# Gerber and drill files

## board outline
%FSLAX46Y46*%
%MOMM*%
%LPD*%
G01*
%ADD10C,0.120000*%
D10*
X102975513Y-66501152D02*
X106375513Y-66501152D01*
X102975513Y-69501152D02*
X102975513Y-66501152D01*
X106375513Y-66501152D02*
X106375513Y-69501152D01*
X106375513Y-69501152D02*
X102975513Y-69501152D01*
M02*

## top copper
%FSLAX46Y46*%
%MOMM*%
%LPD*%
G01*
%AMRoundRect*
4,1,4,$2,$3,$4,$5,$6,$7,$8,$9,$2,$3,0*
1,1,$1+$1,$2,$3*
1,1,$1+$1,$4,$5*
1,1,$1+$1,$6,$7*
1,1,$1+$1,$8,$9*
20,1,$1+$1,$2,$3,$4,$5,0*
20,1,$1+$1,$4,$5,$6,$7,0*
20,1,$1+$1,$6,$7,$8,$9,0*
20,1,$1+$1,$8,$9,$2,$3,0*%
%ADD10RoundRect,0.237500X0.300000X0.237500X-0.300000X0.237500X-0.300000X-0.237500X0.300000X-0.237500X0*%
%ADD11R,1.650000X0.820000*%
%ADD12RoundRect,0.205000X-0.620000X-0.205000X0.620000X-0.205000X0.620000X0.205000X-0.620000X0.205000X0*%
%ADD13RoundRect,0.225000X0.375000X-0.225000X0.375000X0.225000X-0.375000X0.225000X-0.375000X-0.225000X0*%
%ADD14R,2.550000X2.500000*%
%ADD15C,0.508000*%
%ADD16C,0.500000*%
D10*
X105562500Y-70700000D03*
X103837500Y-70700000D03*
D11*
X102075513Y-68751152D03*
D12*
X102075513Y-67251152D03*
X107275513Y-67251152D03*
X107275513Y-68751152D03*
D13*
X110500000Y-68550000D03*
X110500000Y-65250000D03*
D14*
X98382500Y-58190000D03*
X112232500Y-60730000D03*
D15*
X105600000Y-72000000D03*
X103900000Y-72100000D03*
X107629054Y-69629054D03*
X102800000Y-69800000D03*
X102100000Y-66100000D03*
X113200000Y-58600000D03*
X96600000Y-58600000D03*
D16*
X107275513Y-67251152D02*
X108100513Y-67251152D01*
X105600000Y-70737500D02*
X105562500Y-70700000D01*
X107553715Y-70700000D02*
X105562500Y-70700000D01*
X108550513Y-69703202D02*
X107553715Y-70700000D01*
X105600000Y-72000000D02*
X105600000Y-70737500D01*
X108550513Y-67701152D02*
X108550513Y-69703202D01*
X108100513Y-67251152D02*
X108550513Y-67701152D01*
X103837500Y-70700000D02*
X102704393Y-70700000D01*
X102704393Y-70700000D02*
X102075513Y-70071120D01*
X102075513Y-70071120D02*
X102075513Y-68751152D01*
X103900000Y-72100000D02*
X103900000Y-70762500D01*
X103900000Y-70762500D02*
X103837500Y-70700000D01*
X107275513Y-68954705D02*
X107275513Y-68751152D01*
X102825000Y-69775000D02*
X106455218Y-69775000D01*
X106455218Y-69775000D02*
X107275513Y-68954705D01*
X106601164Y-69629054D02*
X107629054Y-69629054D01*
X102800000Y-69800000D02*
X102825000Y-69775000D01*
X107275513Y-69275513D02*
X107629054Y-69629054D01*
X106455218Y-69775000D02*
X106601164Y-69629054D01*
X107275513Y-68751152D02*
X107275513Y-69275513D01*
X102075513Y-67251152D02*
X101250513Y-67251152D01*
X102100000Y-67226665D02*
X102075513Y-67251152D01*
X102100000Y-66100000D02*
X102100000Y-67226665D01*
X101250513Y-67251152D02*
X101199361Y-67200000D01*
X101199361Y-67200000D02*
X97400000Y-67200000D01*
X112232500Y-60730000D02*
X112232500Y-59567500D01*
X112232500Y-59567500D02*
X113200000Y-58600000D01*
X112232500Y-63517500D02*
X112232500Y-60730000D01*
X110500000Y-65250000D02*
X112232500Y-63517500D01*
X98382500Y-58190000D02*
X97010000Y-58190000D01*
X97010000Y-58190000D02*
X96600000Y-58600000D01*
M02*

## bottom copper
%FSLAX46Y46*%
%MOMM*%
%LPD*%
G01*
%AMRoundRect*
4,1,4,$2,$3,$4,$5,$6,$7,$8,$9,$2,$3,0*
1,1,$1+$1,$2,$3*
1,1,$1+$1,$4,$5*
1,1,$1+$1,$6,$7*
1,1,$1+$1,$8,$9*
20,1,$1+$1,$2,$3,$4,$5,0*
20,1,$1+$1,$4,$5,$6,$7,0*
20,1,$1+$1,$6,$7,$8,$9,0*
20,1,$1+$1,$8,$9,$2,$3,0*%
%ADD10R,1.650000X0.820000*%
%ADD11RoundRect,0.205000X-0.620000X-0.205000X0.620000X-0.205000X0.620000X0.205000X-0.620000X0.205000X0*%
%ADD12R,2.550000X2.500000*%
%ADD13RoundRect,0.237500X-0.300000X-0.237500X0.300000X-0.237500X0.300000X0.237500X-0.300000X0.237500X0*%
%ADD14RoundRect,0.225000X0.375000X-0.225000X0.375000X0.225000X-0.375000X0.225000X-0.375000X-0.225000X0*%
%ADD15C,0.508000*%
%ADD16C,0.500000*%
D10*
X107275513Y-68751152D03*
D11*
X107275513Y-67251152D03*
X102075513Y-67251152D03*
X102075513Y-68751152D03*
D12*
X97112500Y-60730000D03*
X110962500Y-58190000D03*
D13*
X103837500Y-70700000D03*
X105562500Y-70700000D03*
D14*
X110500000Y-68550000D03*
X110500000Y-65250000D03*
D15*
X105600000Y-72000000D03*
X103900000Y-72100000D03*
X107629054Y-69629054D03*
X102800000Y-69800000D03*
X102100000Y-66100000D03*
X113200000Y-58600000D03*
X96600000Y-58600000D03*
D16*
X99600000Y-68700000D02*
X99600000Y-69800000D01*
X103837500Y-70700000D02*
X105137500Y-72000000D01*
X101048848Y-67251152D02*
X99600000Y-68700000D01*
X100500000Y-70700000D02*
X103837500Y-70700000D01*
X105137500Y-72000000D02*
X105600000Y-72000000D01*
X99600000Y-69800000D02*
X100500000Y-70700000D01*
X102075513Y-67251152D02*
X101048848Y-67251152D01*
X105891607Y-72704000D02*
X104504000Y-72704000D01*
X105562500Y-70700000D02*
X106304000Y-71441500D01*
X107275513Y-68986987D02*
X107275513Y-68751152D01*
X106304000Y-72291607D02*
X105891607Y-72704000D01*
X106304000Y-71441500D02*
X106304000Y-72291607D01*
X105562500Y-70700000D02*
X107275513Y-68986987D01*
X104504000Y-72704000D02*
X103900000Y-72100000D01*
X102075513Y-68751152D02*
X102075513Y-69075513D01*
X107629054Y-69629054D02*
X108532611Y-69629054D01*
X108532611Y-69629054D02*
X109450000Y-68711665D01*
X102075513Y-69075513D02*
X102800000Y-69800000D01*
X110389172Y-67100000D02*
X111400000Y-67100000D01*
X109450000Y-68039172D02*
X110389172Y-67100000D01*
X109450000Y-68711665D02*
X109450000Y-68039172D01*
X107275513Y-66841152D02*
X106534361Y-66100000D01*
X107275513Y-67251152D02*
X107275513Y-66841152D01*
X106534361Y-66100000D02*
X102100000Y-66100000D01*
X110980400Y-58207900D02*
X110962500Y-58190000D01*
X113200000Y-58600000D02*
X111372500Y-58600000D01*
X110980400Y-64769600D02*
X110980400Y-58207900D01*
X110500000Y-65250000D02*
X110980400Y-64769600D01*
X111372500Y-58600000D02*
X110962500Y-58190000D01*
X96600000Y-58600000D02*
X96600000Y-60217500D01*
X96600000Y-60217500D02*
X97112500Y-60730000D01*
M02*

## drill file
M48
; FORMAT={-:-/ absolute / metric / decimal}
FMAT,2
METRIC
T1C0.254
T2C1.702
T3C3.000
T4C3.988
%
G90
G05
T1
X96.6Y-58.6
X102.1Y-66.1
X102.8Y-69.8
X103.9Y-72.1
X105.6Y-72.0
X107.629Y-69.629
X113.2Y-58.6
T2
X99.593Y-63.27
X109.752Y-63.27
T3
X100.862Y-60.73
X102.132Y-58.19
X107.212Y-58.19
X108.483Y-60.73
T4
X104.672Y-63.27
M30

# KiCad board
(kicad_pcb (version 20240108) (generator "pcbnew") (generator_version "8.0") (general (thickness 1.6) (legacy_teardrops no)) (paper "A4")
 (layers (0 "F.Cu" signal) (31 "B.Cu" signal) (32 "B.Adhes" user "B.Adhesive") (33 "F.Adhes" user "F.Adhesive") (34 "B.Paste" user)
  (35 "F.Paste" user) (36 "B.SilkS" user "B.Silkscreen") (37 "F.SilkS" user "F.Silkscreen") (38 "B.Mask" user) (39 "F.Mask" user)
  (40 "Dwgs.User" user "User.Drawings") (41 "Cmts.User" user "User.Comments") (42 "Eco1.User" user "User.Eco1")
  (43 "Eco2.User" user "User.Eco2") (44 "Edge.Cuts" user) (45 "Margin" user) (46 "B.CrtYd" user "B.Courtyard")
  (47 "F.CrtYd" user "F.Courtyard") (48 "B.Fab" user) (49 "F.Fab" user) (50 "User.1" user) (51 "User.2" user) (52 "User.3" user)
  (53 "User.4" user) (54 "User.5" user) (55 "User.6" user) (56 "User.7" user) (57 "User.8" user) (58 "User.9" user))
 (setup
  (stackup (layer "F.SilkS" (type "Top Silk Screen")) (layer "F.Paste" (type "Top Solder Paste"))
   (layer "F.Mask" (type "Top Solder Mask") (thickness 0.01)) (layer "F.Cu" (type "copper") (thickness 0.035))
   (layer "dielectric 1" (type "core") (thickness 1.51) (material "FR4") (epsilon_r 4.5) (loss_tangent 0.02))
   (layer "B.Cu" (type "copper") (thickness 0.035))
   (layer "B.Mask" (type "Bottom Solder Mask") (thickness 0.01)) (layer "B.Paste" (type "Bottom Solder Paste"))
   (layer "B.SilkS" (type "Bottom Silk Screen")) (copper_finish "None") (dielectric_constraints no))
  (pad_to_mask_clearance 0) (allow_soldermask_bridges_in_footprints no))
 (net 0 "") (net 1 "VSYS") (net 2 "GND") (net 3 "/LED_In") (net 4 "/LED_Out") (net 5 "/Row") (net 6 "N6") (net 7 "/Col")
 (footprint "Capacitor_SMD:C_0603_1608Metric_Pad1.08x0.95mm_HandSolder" (layer "F.Cu") (at 104.7 70.7 180)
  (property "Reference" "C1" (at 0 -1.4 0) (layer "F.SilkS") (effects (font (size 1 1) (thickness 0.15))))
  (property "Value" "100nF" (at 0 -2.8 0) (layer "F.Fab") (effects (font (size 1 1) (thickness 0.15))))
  (pad "1" smd roundrect (at -0.8625 0 180) (size 1.075 0.95) (layers "F.Cu" "F.Paste" "F.Mask") (roundrect_rratio 0.25) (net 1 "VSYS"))
  (pad "2" smd roundrect (at 0.8625 0 180) (size 1.075 0.95) (layers "F.Cu" "F.Paste" "F.Mask") (roundrect_rratio 0.25) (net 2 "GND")))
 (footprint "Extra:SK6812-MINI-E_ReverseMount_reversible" (layer "F.Cu") (at 104.675513 68.001152)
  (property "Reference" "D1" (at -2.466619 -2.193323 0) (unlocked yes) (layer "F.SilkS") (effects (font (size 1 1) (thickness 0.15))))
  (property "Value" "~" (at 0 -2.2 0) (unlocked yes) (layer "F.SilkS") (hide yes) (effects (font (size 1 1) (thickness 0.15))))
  (fp_line (start -1.7 -1.5) (end 1.7 -1.5) (stroke (width 0.12) (type solid)) (layer "Edge.Cuts"))
  (fp_line (start -1.7 1.5) (end -1.7 -1.5) (stroke (width 0.12) (type solid)) (layer "Edge.Cuts"))
  (fp_line (start 1.7 -1.5) (end 1.7 1.5) (stroke (width 0.12) (type solid)) (layer "Edge.Cuts"))
  (fp_line (start 1.7 1.5) (end -1.7 1.5) (stroke (width 0.12) (type solid)) (layer "Edge.Cuts"))
  (pad "1" smd rect (at -2.6 0.75) (size 1.65 0.82) (layers "F.Cu" "F.Paste" "F.Mask") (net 2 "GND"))
  (pad "1" smd rect (at 2.6 0.75) (size 1.65 0.82) (layers "B.Cu" "B.Paste" "B.Mask") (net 2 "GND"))
  (pad "2" smd roundrect (at -2.6 -0.75) (size 1.65 0.82) (layers "F.Cu" "F.Paste" "F.Mask") (roundrect_rratio 0.25) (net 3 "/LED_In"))
  (pad "2" smd roundrect (at 2.6 -0.75) (size 1.65 0.82) (layers "B.Cu" "B.Paste" "B.Mask") (roundrect_rratio 0.25) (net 3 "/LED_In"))
  (pad "3" smd roundrect (at -2.6 -0.75) (size 1.65 0.82) (layers "B.Cu" "B.Paste" "B.Mask") (roundrect_rratio 0.25) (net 1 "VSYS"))
  (pad "3" smd roundrect (at 2.6 -0.75) (size 1.65 0.82) (layers "F.Cu" "F.Paste" "F.Mask") (roundrect_rratio 0.25) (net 1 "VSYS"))
  (pad "4" smd roundrect (at -2.6 0.75) (size 1.65 0.82) (layers "B.Cu" "B.Paste" "B.Mask") (roundrect_rratio 0.25) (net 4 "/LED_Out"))
  (pad "4" smd roundrect (at 2.6 0.75) (size 1.65 0.82) (layers "F.Cu" "F.Paste" "F.Mask") (roundrect_rratio 0.25) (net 4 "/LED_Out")))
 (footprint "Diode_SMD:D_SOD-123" (layer "F.Cu") (at 110.5 66.9 90)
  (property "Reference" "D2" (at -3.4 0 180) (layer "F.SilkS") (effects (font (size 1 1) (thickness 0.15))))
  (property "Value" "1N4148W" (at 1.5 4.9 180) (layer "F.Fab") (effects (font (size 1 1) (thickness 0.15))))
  (pad "1" smd roundrect (at -1.65 0 90) (size 0.9 1.2) (layers "F.Cu" "F.Paste" "F.Mask") (roundrect_rratio 0.25) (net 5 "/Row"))
  (pad "2" smd roundrect (at 1.65 0 90) (size 0.9 1.2) (layers "F.Cu" "F.Paste" "F.Mask") (roundrect_rratio 0.25) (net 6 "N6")))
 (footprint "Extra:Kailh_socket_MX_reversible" (layer "F.Cu") (at 104.6725 63.27)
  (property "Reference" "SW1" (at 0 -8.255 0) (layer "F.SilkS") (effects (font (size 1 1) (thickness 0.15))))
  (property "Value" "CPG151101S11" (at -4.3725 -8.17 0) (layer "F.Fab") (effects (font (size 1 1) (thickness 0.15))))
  (pad "" np_thru_hole circle (at -5.08 0) (size 1.7018 1.7018) (drill 1.7018) (layers "*.Cu" "*.Mask"))
  (pad "" np_thru_hole circle (at -3.81 -2.54) (size 3 3) (drill 3) (layers "*.Cu" "*.Mask"))
  (pad "" np_thru_hole circle (at -2.54 -5.08 180) (size 3 3) (drill 3) (layers "*.Cu" "*.Mask"))
  (pad "" np_thru_hole circle (at 0 0) (size 3.9878 3.9878) (drill 3.9878) (layers "*.Cu" "*.Mask"))
  (pad "" np_thru_hole circle (at 2.54 -5.08) (size 3 3) (drill 3) (layers "*.Cu" "*.Mask"))
  (pad "" np_thru_hole circle (at 3.81 -2.54 180) (size 3 3) (drill 3) (layers "*.Cu" "*.Mask"))
  (pad "" np_thru_hole circle (at 5.08 0) (size 1.7018 1.7018) (drill 1.7018) (layers "*.Cu" "*.Mask"))
  (pad "1" smd rect (at -7.56 -2.54) (size 2.55 2.5) (layers "B.Cu" "B.Paste" "B.Mask") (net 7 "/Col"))
  (pad "1" smd rect (at -6.29 -5.08 180) (size 2.55 2.5) (layers "F.Cu" "F.Paste" "F.Mask") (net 7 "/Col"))
  (pad "2" smd rect (at 6.29 -5.08) (size 2.55 2.5) (layers "B.Cu" "B.Paste" "B.Mask") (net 6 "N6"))
  (pad "2" smd rect (at 7.56 -2.54 180) (size 2.55 2.5) (layers "F.Cu" "F.Paste" "F.Mask") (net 6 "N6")))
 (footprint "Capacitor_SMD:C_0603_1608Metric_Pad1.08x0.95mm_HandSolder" (layer "B.Cu") (at 104.7 70.7)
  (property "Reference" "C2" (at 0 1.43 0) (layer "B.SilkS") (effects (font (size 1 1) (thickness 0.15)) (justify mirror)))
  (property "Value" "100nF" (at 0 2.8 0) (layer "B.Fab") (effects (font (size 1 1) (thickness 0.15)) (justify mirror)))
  (pad "1" smd roundrect (at -0.8625 0) (size 1.075 0.95) (layers "B.Cu" "B.Paste" "B.Mask") (roundrect_rratio 0.25) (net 1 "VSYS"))
  (pad "2" smd roundrect (at 0.8625 0) (size 1.075 0.95) (layers "B.Cu" "B.Paste" "B.Mask") (roundrect_rratio 0.25) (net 2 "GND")))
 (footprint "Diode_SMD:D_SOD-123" (layer "B.Cu") (at 110.5 66.9 90)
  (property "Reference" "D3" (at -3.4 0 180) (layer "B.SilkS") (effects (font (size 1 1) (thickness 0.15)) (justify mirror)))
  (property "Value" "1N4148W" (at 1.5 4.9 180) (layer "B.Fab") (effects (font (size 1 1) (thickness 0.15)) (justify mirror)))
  (pad "1" smd roundrect (at -1.65 0 90) (size 0.9 1.2) (layers "B.Cu" "B.Paste" "B.Mask") (roundrect_rratio 0.25) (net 5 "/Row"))
  (pad "2" smd roundrect (at 1.65 0 90) (size 0.9 1.2) (layers "B.Cu" "B.Paste" "B.Mask") (roundrect_rratio 0.25) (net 6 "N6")))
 (segment (start 107.275513 67.251152) (end 108.100513 67.251152) (width 0.5) (layer "F.Cu") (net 1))
 (segment (start 105.6 70.7375) (end 105.5625 70.7) (width 0.5) (layer "F.Cu") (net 1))
 (segment (start 107.553715 70.7) (end 105.5625 70.7) (width 0.5) (layer "F.Cu") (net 1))
 (segment (start 108.550513 69.703202) (end 107.553715 70.7) (width 0.5) (layer "F.Cu") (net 1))
 (segment (start 105.6 72) (end 105.6 70.7375) (width 0.5) (layer "F.Cu") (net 1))
 (segment (start 108.550513 67.701152) (end 108.550513 69.703202) (width 0.5) (layer "F.Cu") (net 1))
 (segment (start 108.100513 67.251152) (end 108.550513 67.701152) (width 0.5) (layer "F.Cu") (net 1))
 (via (at 105.6 72) (size 0.508) (drill 0.254) (layers "F.Cu" "B.Cu") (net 1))
 (segment (start 99.6 68.7) (end 99.6 69.8) (width 0.5) (layer "B.Cu") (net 1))
 (segment (start 103.8375 70.7) (end 105.1375 72) (width 0.5) (layer "B.Cu") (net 1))
 (segment (start 101.048848 67.251152) (end 99.6 68.7) (width 0.5) (layer "B.Cu") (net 1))
 (segment (start 100.5 70.7) (end 103.8375 70.7) (width 0.5) (layer "B.Cu") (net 1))
 (segment (start 105.1375 72) (end 105.6 72) (width 0.5) (layer "B.Cu") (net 1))
 (segment (start 99.6 69.8) (end 100.5 70.7) (width 0.5) (layer "B.Cu") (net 1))
 (segment (start 102.075513 67.251152) (end 101.048848 67.251152) (width 0.5) (layer "B.Cu") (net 1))
 (segment (start 103.8375 70.7) (end 102.704393 70.7) (width 0.5) (layer "F.Cu") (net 2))
 (segment (start 102.704393 70.7) (end 102.075513 70.07112) (width 0.5) (layer "F.Cu") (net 2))
 (segment (start 102.075513 70.07112) (end 102.075513 68.751152) (width 0.5) (layer "F.Cu") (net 2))
 (segment (start 103.9 72.1) (end 103.9 70.7625) (width 0.5) (layer "F.Cu") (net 2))
 (segment (start 103.9 70.7625) (end 103.8375 70.7) (width 0.5) (layer "F.Cu") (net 2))
 (via (at 103.9 72.1) (size 0.508) (drill 0.254) (layers "F.Cu" "B.Cu") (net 2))
 (segment (start 105.891607 72.704) (end 104.504 72.704) (width 0.5) (layer "B.Cu") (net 2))
 (segment (start 105.5625 70.7) (end 106.304 71.4415) (width 0.5) (layer "B.Cu") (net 2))
 (segment (start 107.275513 68.986987) (end 107.275513 68.751152) (width 0.5) (layer "B.Cu") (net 2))
 (segment (start 106.304 72.291607) (end 105.891607 72.704) (width 0.5) (layer "B.Cu") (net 2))
 (segment (start 106.304 71.4415) (end 106.304 72.291607) (width 0.5) (layer "B.Cu") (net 2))
 (segment (start 105.5625 70.7) (end 107.275513 68.986987) (width 0.5) (layer "B.Cu") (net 2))
 (segment (start 104.504 72.704) (end 103.9 72.1) (width 0.5) (layer "B.Cu") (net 2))
 (segment (start 107.275513 68.954705) (end 107.275513 68.751152) (width 0.5) (layer "F.Cu") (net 4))
 (segment (start 102.825 69.775) (end 106.455218 69.775) (width 0.5) (layer "F.Cu") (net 4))
 (segment (start 106.455218 69.775) (end 107.275513 68.954705) (width 0.5) (layer "F.Cu") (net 4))
 (segment (start 106.601164 69.629054) (end 107.629054 69.629054) (width 0.5) (layer "F.Cu") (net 4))
 (segment (start 102.8 69.8) (end 102.825 69.775) (width 0.5) (layer "F.Cu") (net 4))
 (segment (start 107.275513 69.275513) (end 107.629054 69.629054) (width 0.5) (layer "F.Cu") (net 4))
 (segment (start 106.455218 69.775) (end 106.601164 69.629054) (width 0.5) (layer "F.Cu") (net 4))
 (segment (start 107.275513 68.751152) (end 107.275513 69.275513) (width 0.5) (layer "F.Cu") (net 4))
 (via (at 107.629054 69.629054) (size 0.508) (drill 0.254) (layers "F.Cu" "B.Cu") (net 4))
 (via (at 102.8 69.8) (size 0.508) (drill 0.254) (layers "F.Cu" "B.Cu") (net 4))
 (segment (start 102.075513 68.751152) (end 102.075513 69.075513) (width 0.5) (layer "B.Cu") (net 4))
 (segment (start 107.629054 69.629054) (end 108.532611 69.629054) (width 0.5) (layer "B.Cu") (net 4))
 (segment (start 108.532611 69.629054) (end 109.45 68.711665) (width 0.5) (layer "B.Cu") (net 4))
 (segment (start 102.075513 69.075513) (end 102.8 69.8) (width 0.5) (layer "B.Cu") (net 4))
 (segment (start 110.389172 67.1) (end 111.4 67.1) (width 0.5) (layer "B.Cu") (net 4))
 (segment (start 109.45 68.039172) (end 110.389172 67.1) (width 0.5) (layer "B.Cu") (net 4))
 (segment (start 109.45 68.711665) (end 109.45 68.039172) (width 0.5) (layer "B.Cu") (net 4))
 (segment (start 102.075513 67.251152) (end 101.250513 67.251152) (width 0.5) (layer "F.Cu") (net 3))
 (segment (start 102.1 67.226665) (end 102.075513 67.251152) (width 0.5) (layer "F.Cu") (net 3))
 (segment (start 102.1 66.1) (end 102.1 67.226665) (width 0.5) (layer "F.Cu") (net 3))
 (segment (start 101.250513 67.251152) (end 101.199361 67.2) (width 0.5) (layer "F.Cu") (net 3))
 (segment (start 101.199361 67.2) (end 97.4 67.2) (width 0.5) (layer "F.Cu") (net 3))
 (via (at 102.1 66.1) (size 0.508) (drill 0.254) (layers "F.Cu" "B.Cu") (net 3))
 (segment (start 107.275513 66.841152) (end 106.534361 66.1) (width 0.5) (layer "B.Cu") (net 3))
 (segment (start 107.275513 67.251152) (end 107.275513 66.841152) (width 0.5) (layer "B.Cu") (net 3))
 (segment (start 106.534361 66.1) (end 102.1 66.1) (width 0.5) (layer "B.Cu") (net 3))
 (segment (start 112.2325 60.73) (end 112.2325 59.5675) (width 0.5) (layer "F.Cu") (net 6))
 (segment (start 112.2325 59.5675) (end 113.2 58.6) (width 0.5) (layer "F.Cu") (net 6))
 (segment (start 112.2325 63.5175) (end 112.2325 60.73) (width 0.5) (layer "F.Cu") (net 6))
 (segment (start 110.5 65.25) (end 112.2325 63.5175) (width 0.5) (layer "F.Cu") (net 6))
 (via (at 113.2 58.6) (size 0.508) (drill 0.254) (layers "F.Cu" "B.Cu") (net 6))
 (segment (start 110.9804 58.2079) (end 110.9625 58.19) (width 0.5) (layer "B.Cu") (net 6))
 (segment (start 113.2 58.6) (end 111.3725 58.6) (width 0.5) (layer "B.Cu") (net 6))
 (segment (start 110.9804 64.7696) (end 110.9804 58.2079) (width 0.5) (layer "B.Cu") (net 6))
 (segment (start 110.5 65.25) (end 110.9804 64.7696) (width 0.5) (layer "B.Cu") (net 6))
 (segment (start 111.3725 58.6) (end 110.9625 58.19) (width 0.5) (layer "B.Cu") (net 6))
 (segment (start 98.3825 58.19) (end 97.01 58.19) (width 0.5) (layer "F.Cu") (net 7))
 (segment (start 97.01 58.19) (end 96.6 58.6) (width 0.5) (layer "F.Cu") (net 7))
 (via (at 96.6 58.6) (size 0.508) (drill 0.254) (layers "F.Cu" "B.Cu") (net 7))
 (segment (start 96.6 58.6) (end 96.6 60.2175) (width 0.5) (layer "B.Cu") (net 7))
 (segment (start 96.6 60.2175) (end 97.1125 60.73) (width 0.5) (layer "B.Cu") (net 7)))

